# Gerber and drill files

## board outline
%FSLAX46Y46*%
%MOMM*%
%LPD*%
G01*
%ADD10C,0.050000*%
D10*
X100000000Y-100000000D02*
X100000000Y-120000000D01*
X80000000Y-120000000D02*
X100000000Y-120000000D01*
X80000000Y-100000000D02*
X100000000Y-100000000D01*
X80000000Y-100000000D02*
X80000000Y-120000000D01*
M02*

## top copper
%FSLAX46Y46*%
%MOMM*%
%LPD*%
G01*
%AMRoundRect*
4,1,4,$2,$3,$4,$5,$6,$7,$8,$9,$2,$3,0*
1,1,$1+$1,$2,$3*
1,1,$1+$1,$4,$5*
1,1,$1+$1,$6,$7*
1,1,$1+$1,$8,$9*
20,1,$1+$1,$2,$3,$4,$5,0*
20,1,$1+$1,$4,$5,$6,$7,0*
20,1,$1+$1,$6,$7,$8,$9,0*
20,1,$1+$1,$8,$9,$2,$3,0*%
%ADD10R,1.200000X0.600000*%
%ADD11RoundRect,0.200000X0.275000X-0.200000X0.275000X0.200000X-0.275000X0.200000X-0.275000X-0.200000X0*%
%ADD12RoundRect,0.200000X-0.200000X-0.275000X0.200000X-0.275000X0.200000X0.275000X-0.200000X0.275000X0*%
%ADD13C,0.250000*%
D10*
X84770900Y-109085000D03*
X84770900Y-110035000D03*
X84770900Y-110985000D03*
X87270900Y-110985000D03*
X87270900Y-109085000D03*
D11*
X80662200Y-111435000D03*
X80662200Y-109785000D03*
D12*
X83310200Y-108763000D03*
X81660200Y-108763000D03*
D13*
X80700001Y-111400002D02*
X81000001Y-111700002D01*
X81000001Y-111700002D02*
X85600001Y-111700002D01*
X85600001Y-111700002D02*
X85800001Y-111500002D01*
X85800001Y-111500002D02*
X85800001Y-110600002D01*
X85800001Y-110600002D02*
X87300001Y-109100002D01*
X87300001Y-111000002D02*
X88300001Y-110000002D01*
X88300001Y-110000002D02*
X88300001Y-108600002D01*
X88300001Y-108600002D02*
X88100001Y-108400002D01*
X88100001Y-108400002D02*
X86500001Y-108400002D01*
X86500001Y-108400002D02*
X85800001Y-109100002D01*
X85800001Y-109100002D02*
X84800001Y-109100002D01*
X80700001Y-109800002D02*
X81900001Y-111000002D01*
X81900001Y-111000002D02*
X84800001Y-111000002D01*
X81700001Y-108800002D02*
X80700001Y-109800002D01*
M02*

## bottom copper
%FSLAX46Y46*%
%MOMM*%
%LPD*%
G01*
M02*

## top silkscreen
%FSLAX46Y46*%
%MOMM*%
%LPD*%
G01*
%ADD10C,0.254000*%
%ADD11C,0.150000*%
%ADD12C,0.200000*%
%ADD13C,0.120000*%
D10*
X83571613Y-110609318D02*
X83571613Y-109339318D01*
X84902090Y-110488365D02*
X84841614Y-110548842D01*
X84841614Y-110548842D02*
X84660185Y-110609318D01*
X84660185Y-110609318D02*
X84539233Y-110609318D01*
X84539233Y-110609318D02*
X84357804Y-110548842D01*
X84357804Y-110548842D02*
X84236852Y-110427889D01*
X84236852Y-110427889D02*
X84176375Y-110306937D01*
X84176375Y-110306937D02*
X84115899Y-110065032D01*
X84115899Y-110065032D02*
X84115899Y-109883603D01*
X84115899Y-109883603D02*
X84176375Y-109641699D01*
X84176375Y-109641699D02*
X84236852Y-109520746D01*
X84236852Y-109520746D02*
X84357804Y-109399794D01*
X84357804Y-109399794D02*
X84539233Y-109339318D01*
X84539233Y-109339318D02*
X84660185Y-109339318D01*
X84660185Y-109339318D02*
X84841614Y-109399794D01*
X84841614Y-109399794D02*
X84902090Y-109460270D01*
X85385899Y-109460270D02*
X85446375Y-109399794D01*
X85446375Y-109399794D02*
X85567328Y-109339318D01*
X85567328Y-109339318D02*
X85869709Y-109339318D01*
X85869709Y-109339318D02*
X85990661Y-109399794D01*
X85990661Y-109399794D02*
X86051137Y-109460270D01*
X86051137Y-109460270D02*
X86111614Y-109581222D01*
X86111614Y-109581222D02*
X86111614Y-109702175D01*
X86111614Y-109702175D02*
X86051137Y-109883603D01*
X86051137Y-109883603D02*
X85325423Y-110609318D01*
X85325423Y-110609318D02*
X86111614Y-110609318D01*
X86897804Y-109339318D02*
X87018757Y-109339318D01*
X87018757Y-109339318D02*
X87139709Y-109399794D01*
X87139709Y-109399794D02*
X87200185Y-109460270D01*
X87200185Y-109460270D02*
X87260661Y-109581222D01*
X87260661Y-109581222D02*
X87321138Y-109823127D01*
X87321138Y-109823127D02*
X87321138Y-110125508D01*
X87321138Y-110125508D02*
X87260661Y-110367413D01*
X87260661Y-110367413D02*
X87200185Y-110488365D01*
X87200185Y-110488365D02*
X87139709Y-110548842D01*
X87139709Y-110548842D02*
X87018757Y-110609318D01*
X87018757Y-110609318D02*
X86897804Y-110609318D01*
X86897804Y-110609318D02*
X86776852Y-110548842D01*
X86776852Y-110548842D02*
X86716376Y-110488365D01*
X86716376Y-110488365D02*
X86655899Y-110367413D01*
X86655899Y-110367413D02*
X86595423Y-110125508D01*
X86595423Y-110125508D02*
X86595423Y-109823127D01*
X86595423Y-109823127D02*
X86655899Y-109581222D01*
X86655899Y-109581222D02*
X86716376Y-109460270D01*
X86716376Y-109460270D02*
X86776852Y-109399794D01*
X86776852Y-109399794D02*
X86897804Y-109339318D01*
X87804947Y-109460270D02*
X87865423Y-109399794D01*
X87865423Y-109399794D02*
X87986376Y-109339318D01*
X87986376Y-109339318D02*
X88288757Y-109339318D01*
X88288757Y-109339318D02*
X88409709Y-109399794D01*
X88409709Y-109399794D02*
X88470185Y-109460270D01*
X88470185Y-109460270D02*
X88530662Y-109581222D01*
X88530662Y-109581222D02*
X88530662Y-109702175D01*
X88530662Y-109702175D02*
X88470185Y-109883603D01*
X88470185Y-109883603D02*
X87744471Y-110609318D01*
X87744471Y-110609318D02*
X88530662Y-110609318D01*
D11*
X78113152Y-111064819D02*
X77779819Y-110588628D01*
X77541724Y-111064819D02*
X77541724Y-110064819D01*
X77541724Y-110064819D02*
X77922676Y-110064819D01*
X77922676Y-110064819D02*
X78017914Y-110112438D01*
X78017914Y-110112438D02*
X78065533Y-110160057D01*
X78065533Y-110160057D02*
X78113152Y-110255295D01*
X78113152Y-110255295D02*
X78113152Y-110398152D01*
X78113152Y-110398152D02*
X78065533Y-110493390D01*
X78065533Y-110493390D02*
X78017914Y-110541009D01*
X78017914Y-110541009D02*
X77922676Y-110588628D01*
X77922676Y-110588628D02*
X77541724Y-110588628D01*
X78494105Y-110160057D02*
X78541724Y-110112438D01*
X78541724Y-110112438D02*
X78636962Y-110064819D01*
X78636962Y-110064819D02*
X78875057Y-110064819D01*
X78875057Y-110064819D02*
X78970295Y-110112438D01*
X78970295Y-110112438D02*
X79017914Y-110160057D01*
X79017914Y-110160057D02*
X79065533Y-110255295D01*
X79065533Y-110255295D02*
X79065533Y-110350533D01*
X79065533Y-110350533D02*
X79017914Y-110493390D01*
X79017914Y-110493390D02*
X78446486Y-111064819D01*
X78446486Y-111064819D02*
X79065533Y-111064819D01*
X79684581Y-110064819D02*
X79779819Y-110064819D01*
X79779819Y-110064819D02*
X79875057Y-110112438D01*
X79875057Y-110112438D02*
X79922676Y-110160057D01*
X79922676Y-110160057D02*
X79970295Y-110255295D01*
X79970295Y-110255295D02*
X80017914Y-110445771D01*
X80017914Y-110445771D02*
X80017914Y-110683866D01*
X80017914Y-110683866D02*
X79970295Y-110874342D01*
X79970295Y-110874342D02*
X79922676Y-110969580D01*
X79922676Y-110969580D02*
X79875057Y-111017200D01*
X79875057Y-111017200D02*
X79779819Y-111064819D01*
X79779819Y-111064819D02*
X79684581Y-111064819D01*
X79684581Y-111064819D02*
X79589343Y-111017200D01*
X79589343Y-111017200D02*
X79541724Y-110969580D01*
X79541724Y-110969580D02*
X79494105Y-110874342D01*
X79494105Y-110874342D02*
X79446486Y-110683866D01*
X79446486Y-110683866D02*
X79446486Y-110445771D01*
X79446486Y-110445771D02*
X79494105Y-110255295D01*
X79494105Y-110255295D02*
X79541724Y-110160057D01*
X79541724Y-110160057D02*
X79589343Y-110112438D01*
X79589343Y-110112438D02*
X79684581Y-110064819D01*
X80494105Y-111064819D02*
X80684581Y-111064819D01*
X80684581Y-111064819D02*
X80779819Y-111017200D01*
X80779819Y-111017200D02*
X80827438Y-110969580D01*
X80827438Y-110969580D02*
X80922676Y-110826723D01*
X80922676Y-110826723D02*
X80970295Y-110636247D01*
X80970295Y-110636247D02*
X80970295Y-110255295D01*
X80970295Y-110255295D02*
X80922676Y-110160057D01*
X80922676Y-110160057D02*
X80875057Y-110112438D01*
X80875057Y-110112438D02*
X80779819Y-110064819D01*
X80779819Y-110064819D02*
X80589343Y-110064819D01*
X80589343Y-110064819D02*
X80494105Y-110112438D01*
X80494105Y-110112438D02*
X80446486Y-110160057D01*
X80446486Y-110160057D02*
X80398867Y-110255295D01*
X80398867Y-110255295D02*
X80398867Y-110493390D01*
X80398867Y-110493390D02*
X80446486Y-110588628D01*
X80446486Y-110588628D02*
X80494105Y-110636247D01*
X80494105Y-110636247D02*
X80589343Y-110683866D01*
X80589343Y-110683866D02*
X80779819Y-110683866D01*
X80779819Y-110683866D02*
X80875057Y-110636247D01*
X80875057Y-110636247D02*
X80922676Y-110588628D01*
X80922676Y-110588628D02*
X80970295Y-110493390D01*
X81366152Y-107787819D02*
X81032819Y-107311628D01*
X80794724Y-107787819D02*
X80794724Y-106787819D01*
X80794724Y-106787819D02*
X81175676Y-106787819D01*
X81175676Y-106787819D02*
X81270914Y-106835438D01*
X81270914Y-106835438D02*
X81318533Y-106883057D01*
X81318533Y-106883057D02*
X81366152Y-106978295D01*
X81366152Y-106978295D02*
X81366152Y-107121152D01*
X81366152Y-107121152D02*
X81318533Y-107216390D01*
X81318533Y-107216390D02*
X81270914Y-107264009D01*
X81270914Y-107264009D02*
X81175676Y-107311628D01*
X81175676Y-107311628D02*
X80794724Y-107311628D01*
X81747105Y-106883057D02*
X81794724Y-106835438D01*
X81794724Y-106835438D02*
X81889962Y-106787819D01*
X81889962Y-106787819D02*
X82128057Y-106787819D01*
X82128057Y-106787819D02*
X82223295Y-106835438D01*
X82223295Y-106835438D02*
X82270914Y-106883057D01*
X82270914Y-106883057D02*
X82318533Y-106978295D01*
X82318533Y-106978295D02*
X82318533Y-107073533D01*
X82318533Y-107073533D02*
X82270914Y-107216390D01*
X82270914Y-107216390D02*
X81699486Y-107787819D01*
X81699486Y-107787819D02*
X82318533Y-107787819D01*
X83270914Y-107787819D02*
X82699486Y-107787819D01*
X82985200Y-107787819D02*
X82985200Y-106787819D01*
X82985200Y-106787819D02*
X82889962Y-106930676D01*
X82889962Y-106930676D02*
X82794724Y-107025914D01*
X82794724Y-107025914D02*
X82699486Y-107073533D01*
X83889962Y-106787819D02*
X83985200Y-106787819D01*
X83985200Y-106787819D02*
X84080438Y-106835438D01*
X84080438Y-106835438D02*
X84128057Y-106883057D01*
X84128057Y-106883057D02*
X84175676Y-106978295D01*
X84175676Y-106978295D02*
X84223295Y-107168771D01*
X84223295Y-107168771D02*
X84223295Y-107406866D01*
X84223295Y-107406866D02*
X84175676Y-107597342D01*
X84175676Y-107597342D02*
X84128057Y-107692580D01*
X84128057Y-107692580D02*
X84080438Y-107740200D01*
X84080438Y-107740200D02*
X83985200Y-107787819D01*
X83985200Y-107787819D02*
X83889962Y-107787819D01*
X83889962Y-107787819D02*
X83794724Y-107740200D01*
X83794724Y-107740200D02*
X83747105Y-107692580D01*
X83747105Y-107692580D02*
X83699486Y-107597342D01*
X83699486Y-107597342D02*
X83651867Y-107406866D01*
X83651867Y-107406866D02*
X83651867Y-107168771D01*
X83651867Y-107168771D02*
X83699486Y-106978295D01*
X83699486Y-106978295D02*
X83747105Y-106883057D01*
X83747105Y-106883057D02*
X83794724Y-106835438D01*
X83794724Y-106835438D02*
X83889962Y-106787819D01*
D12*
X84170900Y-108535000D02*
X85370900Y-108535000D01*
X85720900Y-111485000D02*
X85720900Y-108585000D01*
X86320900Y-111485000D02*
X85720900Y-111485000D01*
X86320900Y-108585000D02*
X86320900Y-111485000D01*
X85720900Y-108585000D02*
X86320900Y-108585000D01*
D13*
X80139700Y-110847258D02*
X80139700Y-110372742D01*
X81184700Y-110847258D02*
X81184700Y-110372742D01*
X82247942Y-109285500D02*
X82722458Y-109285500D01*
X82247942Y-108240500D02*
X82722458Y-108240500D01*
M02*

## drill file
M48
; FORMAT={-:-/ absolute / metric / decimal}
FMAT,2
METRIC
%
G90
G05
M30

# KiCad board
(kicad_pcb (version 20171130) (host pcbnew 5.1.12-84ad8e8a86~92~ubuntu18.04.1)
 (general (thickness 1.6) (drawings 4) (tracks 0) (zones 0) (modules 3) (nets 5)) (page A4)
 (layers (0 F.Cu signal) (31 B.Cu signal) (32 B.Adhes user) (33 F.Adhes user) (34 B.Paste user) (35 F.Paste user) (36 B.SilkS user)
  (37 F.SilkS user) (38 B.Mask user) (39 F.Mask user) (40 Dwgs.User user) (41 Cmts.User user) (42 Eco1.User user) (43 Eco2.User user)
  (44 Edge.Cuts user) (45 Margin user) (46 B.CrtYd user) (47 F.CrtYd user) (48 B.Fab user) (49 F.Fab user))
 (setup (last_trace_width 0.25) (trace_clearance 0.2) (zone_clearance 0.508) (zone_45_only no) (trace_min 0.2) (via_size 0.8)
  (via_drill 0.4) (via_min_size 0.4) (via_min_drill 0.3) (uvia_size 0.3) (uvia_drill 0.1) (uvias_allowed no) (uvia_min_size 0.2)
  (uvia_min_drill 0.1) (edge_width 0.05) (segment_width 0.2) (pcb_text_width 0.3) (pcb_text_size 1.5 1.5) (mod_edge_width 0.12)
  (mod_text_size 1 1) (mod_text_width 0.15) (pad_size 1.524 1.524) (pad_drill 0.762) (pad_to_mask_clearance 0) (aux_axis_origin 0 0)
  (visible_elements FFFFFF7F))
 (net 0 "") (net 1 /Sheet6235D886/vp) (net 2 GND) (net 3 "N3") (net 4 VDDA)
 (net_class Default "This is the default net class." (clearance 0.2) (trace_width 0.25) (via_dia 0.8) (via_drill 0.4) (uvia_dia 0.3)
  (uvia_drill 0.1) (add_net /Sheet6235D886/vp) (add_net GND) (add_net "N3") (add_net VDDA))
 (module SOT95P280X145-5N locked (layer F.Cu) (at 86.020900 110.035000)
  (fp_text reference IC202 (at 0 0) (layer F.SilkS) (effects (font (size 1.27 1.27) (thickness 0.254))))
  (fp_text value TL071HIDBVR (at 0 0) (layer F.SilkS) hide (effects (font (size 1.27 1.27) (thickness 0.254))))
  (fp_line (start -1.85 -1.5) (end -0.65 -1.5) (layer F.SilkS) (width 0.2))
  (fp_line (start -0.3 1.45) (end -0.3 -1.45) (layer F.SilkS) (width 0.2))
  (fp_line (start 0.3 1.45) (end -0.3 1.45) (layer F.SilkS) (width 0.2))
  (fp_line (start 0.3 -1.45) (end 0.3 1.45) (layer F.SilkS) (width 0.2))
  (fp_line (start -0.3 -1.45) (end 0.3 -1.45) (layer F.SilkS) (width 0.2))
  (pad 1 smd rect (at -1.25 -0.95 90.000000) (size 0.6 1.2) (layers F.Cu F.Mask F.Paste) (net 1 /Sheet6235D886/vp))
  (pad 2 smd rect (at -1.25 0 90.000000) (size 0.6 1.2) (layers F.Cu F.Mask F.Paste) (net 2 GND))
  (pad 3 smd rect (at -1.25 0.95 90.000000) (size 0.6 1.2) (layers F.Cu F.Mask F.Paste) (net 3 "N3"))
  (pad 4 smd rect (at 1.25 0.95 90.000000) (size 0.6 1.2) (layers F.Cu F.Mask F.Paste) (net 1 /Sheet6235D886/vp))
  (pad 5 smd rect (at 1.25 -0.95 90.000000) (size 0.6 1.2) (layers F.Cu F.Mask F.Paste) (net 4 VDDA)))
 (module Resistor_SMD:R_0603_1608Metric (layer F.Cu) (at 80.662200 110.610000 90.000000)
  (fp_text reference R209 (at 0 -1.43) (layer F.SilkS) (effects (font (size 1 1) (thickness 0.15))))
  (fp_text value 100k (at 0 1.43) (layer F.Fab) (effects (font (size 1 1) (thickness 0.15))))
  (fp_line (start -0.237258 -0.5225) (end 0.237258 -0.5225) (layer F.SilkS) (width 0.12))
  (fp_line (start -0.237258 0.5225) (end 0.237258 0.5225) (layer F.SilkS) (width 0.12))
  (pad 1 smd roundrect (at -0.825 0 90.000000) (size 0.8 0.95) (layers F.Cu F.Mask F.Paste) (roundrect_rratio 0.25) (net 4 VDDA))
  (pad 2 smd roundrect (at 0.825 0 90.000000) (size 0.8 0.95) (layers F.Cu F.Mask F.Paste) (roundrect_rratio 0.25) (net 3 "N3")))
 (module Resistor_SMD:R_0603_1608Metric (layer F.Cu) (at 82.485200 108.763000)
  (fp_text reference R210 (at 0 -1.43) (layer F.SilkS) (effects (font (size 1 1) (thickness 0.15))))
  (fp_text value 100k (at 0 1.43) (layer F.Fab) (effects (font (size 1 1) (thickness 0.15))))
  (fp_line (start -0.237258 0.5225) (end 0.237258 0.5225) (layer F.SilkS) (width 0.12))
  (fp_line (start -0.237258 -0.5225) (end 0.237258 -0.5225) (layer F.SilkS) (width 0.12))
  (pad 2 smd roundrect (at 0.825 0) (size 0.8 0.95) (layers F.Cu F.Mask F.Paste) (roundrect_rratio 0.25) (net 2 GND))
  (pad 1 smd roundrect (at -0.825 0) (size 0.8 0.95) (layers F.Cu F.Mask F.Paste) (roundrect_rratio 0.25) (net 3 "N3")))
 (gr_line (start 100 100) (end 100 120) (layer Edge.Cuts) (width 0.05))
 (gr_line (start 80 120) (end 100 120) (layer Edge.Cuts) (width 0.05))
 (gr_line (start 80 100) (end 100 100) (layer Edge.Cuts) (width 0.05))
 (gr_line (start 80 100) (end 80 120) (layer Edge.Cuts) (width 0.05))
 (segment (start 80.700001 111.400002) (end 81.000001 111.700002) (width 0.250000) (layer F.Cu) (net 4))
 (segment (start 81.000001 111.700002) (end 85.600001 111.700002) (width 0.250000) (layer F.Cu) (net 4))
 (segment (start 85.600001 111.700002) (end 85.800001 111.500002) (width 0.250000) (layer F.Cu) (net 4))
 (segment (start 85.800001 111.500002) (end 85.800001 110.600002) (width 0.250000) (layer F.Cu) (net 4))
 (segment (start 85.800001 110.600002) (end 87.300001 109.100002) (width 0.250000) (layer F.Cu) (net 4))
 (segment (start 87.300001 111.000002) (end 88.300001 110.000002) (width 0.250000) (layer F.Cu) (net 1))
 (segment (start 88.300001 110.000002) (end 88.300001 108.600002) (width 0.250000) (layer F.Cu) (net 1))
 (segment (start 88.300001 108.600002) (end 88.100001 108.400002) (width 0.250000) (layer F.Cu) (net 1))
 (segment (start 88.100001 108.400002) (end 86.500001 108.400002) (width 0.250000) (layer F.Cu) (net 1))
 (segment (start 86.500001 108.400002) (end 85.800001 109.100002) (width 0.250000) (layer F.Cu) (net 1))
 (segment (start 85.800001 109.100002) (end 84.800001 109.100002) (width 0.250000) (layer F.Cu) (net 1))
 (segment (start 80.700001 109.800002) (end 81.900001 111.000002) (width 0.250000) (layer F.Cu) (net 3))
 (segment (start 81.900001 111.000002) (end 84.800001 111.000002) (width 0.250000) (layer F.Cu) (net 3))
 (segment (start 81.700001 108.800002) (end 80.700001 109.800002) (width 0.250000) (layer F.Cu) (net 3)))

